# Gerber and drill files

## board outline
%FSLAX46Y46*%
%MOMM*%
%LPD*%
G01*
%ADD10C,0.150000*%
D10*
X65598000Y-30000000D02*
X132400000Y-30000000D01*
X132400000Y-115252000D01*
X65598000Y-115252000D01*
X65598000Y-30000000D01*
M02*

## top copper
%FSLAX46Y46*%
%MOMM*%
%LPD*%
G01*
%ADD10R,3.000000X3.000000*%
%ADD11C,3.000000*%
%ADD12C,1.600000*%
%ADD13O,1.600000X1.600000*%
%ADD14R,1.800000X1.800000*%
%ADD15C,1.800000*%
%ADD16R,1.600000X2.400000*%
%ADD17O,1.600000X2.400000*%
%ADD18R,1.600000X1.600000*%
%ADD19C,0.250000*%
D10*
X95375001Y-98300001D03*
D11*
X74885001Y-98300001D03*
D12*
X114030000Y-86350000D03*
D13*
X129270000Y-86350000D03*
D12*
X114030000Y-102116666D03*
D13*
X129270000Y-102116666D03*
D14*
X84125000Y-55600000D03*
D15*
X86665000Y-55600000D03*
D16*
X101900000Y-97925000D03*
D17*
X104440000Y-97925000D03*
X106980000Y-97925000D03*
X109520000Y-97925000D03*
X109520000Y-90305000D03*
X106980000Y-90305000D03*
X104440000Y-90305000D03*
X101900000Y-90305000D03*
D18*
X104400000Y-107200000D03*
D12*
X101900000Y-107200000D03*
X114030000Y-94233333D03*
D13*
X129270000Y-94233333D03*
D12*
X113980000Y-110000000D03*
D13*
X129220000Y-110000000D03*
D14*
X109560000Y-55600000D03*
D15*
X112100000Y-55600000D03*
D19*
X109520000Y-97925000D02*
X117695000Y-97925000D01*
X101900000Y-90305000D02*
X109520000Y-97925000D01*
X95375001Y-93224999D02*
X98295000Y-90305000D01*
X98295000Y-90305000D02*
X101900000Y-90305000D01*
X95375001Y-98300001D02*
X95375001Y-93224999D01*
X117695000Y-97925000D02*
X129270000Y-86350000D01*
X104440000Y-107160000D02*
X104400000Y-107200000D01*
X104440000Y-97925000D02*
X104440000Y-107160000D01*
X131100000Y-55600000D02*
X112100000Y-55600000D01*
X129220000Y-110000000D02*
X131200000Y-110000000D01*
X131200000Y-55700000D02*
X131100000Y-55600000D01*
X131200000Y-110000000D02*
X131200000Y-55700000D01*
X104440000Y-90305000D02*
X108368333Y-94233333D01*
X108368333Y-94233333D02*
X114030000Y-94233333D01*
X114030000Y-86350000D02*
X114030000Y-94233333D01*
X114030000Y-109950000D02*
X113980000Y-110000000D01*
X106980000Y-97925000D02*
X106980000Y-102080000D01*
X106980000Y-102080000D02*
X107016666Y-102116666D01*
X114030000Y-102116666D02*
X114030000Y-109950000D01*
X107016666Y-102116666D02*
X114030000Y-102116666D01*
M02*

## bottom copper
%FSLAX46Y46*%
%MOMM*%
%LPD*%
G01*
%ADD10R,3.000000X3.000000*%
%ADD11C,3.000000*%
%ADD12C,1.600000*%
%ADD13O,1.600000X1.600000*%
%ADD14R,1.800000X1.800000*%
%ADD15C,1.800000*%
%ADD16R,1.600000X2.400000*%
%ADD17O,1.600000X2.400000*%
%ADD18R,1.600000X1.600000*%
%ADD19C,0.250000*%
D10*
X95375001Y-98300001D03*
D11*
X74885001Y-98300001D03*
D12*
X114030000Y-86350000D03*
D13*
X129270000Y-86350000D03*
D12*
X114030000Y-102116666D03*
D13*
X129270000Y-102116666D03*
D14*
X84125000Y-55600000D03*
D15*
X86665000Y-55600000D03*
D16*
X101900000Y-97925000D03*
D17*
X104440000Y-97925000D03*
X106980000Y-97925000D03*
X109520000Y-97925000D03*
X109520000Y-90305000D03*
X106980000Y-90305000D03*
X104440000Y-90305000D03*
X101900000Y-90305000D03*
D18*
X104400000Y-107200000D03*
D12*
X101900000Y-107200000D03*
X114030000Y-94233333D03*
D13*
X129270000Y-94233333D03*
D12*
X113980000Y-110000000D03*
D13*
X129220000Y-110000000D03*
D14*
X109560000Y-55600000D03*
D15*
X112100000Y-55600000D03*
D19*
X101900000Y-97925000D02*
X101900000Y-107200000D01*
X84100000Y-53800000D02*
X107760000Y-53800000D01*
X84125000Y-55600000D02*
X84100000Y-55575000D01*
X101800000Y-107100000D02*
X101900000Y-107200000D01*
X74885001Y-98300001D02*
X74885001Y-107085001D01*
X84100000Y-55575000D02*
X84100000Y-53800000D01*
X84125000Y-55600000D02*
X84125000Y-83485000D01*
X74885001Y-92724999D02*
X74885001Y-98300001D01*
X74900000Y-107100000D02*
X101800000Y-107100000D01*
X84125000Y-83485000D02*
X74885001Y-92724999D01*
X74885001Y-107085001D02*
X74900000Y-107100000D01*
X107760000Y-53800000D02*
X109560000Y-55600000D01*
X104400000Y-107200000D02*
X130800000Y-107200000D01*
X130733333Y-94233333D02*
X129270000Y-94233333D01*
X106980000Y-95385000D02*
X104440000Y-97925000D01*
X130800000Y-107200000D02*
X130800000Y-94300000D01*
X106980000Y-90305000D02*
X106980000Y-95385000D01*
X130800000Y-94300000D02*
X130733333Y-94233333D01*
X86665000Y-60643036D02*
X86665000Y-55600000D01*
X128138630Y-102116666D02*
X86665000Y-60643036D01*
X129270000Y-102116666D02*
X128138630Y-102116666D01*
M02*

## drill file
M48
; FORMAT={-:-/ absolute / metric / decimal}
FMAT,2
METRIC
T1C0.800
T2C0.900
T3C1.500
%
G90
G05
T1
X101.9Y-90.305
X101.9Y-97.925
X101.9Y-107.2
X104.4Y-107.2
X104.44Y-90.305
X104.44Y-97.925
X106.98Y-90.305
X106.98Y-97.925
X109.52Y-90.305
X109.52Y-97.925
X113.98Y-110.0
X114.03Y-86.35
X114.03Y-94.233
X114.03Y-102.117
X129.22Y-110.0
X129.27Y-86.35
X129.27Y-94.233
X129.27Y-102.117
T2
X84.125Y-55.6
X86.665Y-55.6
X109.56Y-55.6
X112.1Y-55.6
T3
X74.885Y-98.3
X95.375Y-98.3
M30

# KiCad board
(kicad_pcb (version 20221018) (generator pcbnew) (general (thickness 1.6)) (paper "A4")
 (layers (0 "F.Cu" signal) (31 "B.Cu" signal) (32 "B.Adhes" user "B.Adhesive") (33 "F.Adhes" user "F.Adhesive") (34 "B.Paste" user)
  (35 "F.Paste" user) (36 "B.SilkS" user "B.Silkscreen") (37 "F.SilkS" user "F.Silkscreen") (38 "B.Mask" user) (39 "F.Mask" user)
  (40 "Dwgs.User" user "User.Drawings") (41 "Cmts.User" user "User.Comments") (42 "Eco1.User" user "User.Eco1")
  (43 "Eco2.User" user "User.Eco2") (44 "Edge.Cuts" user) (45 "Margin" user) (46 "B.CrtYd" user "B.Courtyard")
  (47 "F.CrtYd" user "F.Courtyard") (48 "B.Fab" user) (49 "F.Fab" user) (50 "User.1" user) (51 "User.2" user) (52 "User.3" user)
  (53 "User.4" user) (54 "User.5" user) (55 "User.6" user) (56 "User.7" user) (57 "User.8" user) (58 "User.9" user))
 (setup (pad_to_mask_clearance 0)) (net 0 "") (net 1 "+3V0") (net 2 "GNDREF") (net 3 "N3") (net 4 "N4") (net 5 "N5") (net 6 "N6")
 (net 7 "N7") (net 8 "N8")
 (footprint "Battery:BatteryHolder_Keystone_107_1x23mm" (layer "F.Cu") (at 95.375001 98.300001 180)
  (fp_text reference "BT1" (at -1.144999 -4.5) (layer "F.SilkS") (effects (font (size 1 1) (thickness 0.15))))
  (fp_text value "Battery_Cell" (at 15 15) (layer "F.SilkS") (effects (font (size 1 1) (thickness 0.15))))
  (pad "1" thru_hole rect (at 0 0 180) (size 3 3) (drill 1.5) (layers "*.Cu" "*.Mask") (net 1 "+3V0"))
  (pad "2" thru_hole circle (at 20.49 0 180) (size 3 3) (drill 1.5) (layers "*.Cu" "*.Mask") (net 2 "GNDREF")))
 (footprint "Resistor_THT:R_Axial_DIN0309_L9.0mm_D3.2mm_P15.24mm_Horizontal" (layer "F.Cu") (at 114.03 86.35)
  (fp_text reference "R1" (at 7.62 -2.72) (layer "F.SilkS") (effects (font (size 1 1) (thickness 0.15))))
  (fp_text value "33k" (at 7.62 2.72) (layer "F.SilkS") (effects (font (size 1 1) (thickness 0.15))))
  (pad "1" thru_hole circle (at 0 0) (size 1.6 1.6) (drill 0.8) (layers "*.Cu" "*.Mask") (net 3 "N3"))
  (pad "2" thru_hole oval (at 15.24 0) (size 1.6 1.6) (drill 0.8) (layers "*.Cu" "*.Mask") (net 1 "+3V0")))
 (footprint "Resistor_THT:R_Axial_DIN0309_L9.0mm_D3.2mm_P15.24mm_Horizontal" (layer "F.Cu") (at 114.03 102.116666)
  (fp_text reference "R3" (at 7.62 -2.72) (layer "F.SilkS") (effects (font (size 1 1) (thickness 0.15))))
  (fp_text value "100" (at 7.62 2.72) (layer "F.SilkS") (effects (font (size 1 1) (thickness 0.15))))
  (pad "1" thru_hole circle (at 0 0) (size 1.6 1.6) (drill 0.8) (layers "*.Cu" "*.Mask") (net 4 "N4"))
  (pad "2" thru_hole oval (at 15.24 0) (size 1.6 1.6) (drill 0.8) (layers "*.Cu" "*.Mask") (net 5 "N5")))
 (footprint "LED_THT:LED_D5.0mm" (layer "F.Cu") (at 84.125 55.6)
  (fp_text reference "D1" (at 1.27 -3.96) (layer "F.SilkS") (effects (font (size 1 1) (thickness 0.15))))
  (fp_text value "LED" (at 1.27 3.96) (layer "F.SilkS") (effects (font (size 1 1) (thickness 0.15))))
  (pad "1" thru_hole rect (at 0 0) (size 1.8 1.8) (drill 0.9) (layers "*.Cu" "*.Mask") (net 2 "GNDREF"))
  (pad "2" thru_hole circle (at 2.54 0) (size 1.8 1.8) (drill 0.9) (layers "*.Cu" "*.Mask") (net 5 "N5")))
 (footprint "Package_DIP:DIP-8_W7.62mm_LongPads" (layer "F.Cu") (at 101.9 97.925 90)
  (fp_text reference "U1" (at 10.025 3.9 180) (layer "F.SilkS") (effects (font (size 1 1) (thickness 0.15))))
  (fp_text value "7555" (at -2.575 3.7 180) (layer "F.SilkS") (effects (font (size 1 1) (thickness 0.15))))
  (pad "1" thru_hole rect (at 0 0 90) (size 2.4 1.6) (drill 0.8) (layers "*.Cu" "*.Mask") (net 2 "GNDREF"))
  (pad "2" thru_hole oval (at 0 2.54 90) (size 2.4 1.6) (drill 0.8) (layers "*.Cu" "*.Mask") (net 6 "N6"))
  (pad "3" thru_hole oval (at 0 5.08 90) (size 2.4 1.6) (drill 0.8) (layers "*.Cu" "*.Mask") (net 4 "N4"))
  (pad "4" thru_hole oval (at 0 7.62 90) (size 2.4 1.6) (drill 0.8) (layers "*.Cu" "*.Mask") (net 1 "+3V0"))
  (pad "5" thru_hole oval (at 7.62 7.62 90) (size 2.4 1.6) (drill 0.8) (layers "*.Cu" "*.Mask") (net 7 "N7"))
  (pad "6" thru_hole oval (at 7.62 5.08 90) (size 2.4 1.6) (drill 0.8) (layers "*.Cu" "*.Mask") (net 6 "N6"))
  (pad "7" thru_hole oval (at 7.62 2.54 90) (size 2.4 1.6) (drill 0.8) (layers "*.Cu" "*.Mask") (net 3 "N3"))
  (pad "8" thru_hole oval (at 7.62 0 90) (size 2.4 1.6) (drill 0.8) (layers "*.Cu" "*.Mask") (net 1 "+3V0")))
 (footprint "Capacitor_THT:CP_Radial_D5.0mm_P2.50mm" (layer "F.Cu") (at 104.4 107.2 180)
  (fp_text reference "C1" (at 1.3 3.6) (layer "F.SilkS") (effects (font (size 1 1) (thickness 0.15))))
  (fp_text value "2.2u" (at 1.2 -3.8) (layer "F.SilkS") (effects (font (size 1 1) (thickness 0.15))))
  (pad "1" thru_hole rect (at 0 0 180) (size 1.6 1.6) (drill 0.8) (layers "*.Cu" "*.Mask") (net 6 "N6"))
  (pad "2" thru_hole circle (at 2.5 0 180) (size 1.6 1.6) (drill 0.8) (layers "*.Cu" "*.Mask") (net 2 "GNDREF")))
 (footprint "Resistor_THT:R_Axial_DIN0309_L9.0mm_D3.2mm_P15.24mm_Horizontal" (layer "F.Cu") (at 114.03 94.233333)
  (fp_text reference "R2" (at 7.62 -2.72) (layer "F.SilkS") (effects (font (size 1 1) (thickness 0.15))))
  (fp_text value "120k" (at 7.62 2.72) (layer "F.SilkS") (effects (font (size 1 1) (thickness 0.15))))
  (pad "1" thru_hole circle (at 0 0) (size 1.6 1.6) (drill 0.8) (layers "*.Cu" "*.Mask") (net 3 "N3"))
  (pad "2" thru_hole oval (at 15.24 0) (size 1.6 1.6) (drill 0.8) (layers "*.Cu" "*.Mask") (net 6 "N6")))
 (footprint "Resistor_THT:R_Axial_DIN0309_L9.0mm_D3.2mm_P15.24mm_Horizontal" (layer "F.Cu") (at 113.98 110)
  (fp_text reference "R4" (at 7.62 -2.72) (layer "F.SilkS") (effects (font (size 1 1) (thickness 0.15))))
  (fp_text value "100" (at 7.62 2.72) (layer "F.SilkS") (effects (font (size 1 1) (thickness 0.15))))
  (pad "1" thru_hole circle (at 0 0) (size 1.6 1.6) (drill 0.8) (layers "*.Cu" "*.Mask") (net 4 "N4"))
  (pad "2" thru_hole oval (at 15.24 0) (size 1.6 1.6) (drill 0.8) (layers "*.Cu" "*.Mask") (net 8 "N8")))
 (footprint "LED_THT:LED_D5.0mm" (layer "F.Cu") (at 109.56 55.6)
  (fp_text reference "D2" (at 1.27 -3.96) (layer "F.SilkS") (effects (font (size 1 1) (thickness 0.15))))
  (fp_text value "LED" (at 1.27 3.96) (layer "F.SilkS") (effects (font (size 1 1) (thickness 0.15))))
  (pad "1" thru_hole rect (at 0 0) (size 1.8 1.8) (drill 0.9) (layers "*.Cu" "*.Mask") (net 2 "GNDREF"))
  (pad "2" thru_hole circle (at 2.54 0) (size 1.8 1.8) (drill 0.9) (layers "*.Cu" "*.Mask") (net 8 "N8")))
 (gr_rect (start 65.598 30) (end 132.4 115.252) (stroke (width 0.15) (type default)) (fill none) (layer "Edge.Cuts"))
 (segment (start 101.9 97.925) (end 101.9 107.2) (width 0.25) (layer "B.Cu") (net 2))
 (segment (start 84.1 53.8) (end 107.76 53.8) (width 0.25) (layer "B.Cu") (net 2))
 (segment (start 84.125 55.6) (end 84.1 55.575) (width 0.25) (layer "B.Cu") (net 2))
 (segment (start 101.8 107.1) (end 101.9 107.2) (width 0.25) (layer "B.Cu") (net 2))
 (segment (start 74.885001 98.300001) (end 74.885001 107.085001) (width 0.25) (layer "B.Cu") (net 2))
 (segment (start 84.1 55.575) (end 84.1 53.8) (width 0.25) (layer "B.Cu") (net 2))
 (segment (start 84.125 55.6) (end 84.125 83.485) (width 0.25) (layer "B.Cu") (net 2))
 (segment (start 74.885001 92.724999) (end 74.885001 98.300001) (width 0.25) (layer "B.Cu") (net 2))
 (segment (start 74.9 107.1) (end 101.8 107.1) (width 0.25) (layer "B.Cu") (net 2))
 (segment (start 84.125 83.485) (end 74.885001 92.724999) (width 0.25) (layer "B.Cu") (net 2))
 (segment (start 74.885001 107.085001) (end 74.9 107.1) (width 0.25) (layer "B.Cu") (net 2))
 (segment (start 107.76 53.8) (end 109.56 55.6) (width 0.25) (layer "B.Cu") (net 2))
 (segment (start 109.52 97.925) (end 117.695 97.925) (width 0.25) (layer "F.Cu") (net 1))
 (segment (start 101.9 90.305) (end 109.52 97.925) (width 0.25) (layer "F.Cu") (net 1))
 (segment (start 95.375001 93.224999) (end 98.295 90.305) (width 0.25) (layer "F.Cu") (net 1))
 (segment (start 98.295 90.305) (end 101.9 90.305) (width 0.25) (layer "F.Cu") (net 1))
 (segment (start 95.375001 98.300001) (end 95.375001 93.224999) (width 0.25) (layer "F.Cu") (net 1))
 (segment (start 117.695 97.925) (end 129.27 86.35) (width 0.25) (layer "F.Cu") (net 1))
 (segment (start 104.44 107.16) (end 104.4 107.2) (width 0.25) (layer "F.Cu") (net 6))
 (segment (start 104.44 97.925) (end 104.44 107.16) (width 0.25) (layer "F.Cu") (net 6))
 (segment (start 104.4 107.2) (end 130.8 107.2) (width 0.25) (layer "B.Cu") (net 6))
 (segment (start 130.733333 94.233333) (end 129.27 94.233333) (width 0.25) (layer "B.Cu") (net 6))
 (segment (start 106.98 95.385) (end 104.44 97.925) (width 0.25) (layer "B.Cu") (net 6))
 (segment (start 130.8 107.2) (end 130.8 94.3) (width 0.25) (layer "B.Cu") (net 6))
 (segment (start 106.98 90.305) (end 106.98 95.385) (width 0.25) (layer "B.Cu") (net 6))
 (segment (start 130.8 94.3) (end 130.733333 94.233333) (width 0.25) (layer "B.Cu") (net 6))
 (segment (start 86.665 60.643036) (end 86.665 55.6) (width 0.25) (layer "B.Cu") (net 5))
 (segment (start 128.13863 102.116666) (end 86.665 60.643036) (width 0.25) (layer "B.Cu") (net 5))
 (segment (start 129.27 102.116666) (end 128.13863 102.116666) (width 0.25) (layer "B.Cu") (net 5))
 (segment (start 131.1 55.6) (end 112.1 55.6) (width 0.25) (layer "F.Cu") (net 8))
 (segment (start 129.22 110) (end 131.2 110) (width 0.25) (layer "F.Cu") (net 8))
 (segment (start 131.2 55.7) (end 131.1 55.6) (width 0.25) (layer "F.Cu") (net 8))
 (segment (start 131.2 110) (end 131.2 55.7) (width 0.25) (layer "F.Cu") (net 8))
 (segment (start 104.44 90.305) (end 108.368333 94.233333) (width 0.25) (layer "F.Cu") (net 3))
 (segment (start 108.368333 94.233333) (end 114.03 94.233333) (width 0.25) (layer "F.Cu") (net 3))
 (segment (start 114.03 86.35) (end 114.03 94.233333) (width 0.25) (layer "F.Cu") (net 3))
 (segment (start 114.03 109.95) (end 113.98 110) (width 0.25) (layer "F.Cu") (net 4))
 (segment (start 106.98 97.925) (end 106.98 102.08) (width 0.25) (layer "F.Cu") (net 4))
 (segment (start 106.98 102.08) (end 107.016666 102.116666) (width 0.25) (layer "F.Cu") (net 4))
 (segment (start 114.03 102.116666) (end 114.03 109.95) (width 0.25) (layer "F.Cu") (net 4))
 (segment (start 107.016666 102.116666) (end 114.03 102.116666) (width 0.25) (layer "F.Cu") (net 4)))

